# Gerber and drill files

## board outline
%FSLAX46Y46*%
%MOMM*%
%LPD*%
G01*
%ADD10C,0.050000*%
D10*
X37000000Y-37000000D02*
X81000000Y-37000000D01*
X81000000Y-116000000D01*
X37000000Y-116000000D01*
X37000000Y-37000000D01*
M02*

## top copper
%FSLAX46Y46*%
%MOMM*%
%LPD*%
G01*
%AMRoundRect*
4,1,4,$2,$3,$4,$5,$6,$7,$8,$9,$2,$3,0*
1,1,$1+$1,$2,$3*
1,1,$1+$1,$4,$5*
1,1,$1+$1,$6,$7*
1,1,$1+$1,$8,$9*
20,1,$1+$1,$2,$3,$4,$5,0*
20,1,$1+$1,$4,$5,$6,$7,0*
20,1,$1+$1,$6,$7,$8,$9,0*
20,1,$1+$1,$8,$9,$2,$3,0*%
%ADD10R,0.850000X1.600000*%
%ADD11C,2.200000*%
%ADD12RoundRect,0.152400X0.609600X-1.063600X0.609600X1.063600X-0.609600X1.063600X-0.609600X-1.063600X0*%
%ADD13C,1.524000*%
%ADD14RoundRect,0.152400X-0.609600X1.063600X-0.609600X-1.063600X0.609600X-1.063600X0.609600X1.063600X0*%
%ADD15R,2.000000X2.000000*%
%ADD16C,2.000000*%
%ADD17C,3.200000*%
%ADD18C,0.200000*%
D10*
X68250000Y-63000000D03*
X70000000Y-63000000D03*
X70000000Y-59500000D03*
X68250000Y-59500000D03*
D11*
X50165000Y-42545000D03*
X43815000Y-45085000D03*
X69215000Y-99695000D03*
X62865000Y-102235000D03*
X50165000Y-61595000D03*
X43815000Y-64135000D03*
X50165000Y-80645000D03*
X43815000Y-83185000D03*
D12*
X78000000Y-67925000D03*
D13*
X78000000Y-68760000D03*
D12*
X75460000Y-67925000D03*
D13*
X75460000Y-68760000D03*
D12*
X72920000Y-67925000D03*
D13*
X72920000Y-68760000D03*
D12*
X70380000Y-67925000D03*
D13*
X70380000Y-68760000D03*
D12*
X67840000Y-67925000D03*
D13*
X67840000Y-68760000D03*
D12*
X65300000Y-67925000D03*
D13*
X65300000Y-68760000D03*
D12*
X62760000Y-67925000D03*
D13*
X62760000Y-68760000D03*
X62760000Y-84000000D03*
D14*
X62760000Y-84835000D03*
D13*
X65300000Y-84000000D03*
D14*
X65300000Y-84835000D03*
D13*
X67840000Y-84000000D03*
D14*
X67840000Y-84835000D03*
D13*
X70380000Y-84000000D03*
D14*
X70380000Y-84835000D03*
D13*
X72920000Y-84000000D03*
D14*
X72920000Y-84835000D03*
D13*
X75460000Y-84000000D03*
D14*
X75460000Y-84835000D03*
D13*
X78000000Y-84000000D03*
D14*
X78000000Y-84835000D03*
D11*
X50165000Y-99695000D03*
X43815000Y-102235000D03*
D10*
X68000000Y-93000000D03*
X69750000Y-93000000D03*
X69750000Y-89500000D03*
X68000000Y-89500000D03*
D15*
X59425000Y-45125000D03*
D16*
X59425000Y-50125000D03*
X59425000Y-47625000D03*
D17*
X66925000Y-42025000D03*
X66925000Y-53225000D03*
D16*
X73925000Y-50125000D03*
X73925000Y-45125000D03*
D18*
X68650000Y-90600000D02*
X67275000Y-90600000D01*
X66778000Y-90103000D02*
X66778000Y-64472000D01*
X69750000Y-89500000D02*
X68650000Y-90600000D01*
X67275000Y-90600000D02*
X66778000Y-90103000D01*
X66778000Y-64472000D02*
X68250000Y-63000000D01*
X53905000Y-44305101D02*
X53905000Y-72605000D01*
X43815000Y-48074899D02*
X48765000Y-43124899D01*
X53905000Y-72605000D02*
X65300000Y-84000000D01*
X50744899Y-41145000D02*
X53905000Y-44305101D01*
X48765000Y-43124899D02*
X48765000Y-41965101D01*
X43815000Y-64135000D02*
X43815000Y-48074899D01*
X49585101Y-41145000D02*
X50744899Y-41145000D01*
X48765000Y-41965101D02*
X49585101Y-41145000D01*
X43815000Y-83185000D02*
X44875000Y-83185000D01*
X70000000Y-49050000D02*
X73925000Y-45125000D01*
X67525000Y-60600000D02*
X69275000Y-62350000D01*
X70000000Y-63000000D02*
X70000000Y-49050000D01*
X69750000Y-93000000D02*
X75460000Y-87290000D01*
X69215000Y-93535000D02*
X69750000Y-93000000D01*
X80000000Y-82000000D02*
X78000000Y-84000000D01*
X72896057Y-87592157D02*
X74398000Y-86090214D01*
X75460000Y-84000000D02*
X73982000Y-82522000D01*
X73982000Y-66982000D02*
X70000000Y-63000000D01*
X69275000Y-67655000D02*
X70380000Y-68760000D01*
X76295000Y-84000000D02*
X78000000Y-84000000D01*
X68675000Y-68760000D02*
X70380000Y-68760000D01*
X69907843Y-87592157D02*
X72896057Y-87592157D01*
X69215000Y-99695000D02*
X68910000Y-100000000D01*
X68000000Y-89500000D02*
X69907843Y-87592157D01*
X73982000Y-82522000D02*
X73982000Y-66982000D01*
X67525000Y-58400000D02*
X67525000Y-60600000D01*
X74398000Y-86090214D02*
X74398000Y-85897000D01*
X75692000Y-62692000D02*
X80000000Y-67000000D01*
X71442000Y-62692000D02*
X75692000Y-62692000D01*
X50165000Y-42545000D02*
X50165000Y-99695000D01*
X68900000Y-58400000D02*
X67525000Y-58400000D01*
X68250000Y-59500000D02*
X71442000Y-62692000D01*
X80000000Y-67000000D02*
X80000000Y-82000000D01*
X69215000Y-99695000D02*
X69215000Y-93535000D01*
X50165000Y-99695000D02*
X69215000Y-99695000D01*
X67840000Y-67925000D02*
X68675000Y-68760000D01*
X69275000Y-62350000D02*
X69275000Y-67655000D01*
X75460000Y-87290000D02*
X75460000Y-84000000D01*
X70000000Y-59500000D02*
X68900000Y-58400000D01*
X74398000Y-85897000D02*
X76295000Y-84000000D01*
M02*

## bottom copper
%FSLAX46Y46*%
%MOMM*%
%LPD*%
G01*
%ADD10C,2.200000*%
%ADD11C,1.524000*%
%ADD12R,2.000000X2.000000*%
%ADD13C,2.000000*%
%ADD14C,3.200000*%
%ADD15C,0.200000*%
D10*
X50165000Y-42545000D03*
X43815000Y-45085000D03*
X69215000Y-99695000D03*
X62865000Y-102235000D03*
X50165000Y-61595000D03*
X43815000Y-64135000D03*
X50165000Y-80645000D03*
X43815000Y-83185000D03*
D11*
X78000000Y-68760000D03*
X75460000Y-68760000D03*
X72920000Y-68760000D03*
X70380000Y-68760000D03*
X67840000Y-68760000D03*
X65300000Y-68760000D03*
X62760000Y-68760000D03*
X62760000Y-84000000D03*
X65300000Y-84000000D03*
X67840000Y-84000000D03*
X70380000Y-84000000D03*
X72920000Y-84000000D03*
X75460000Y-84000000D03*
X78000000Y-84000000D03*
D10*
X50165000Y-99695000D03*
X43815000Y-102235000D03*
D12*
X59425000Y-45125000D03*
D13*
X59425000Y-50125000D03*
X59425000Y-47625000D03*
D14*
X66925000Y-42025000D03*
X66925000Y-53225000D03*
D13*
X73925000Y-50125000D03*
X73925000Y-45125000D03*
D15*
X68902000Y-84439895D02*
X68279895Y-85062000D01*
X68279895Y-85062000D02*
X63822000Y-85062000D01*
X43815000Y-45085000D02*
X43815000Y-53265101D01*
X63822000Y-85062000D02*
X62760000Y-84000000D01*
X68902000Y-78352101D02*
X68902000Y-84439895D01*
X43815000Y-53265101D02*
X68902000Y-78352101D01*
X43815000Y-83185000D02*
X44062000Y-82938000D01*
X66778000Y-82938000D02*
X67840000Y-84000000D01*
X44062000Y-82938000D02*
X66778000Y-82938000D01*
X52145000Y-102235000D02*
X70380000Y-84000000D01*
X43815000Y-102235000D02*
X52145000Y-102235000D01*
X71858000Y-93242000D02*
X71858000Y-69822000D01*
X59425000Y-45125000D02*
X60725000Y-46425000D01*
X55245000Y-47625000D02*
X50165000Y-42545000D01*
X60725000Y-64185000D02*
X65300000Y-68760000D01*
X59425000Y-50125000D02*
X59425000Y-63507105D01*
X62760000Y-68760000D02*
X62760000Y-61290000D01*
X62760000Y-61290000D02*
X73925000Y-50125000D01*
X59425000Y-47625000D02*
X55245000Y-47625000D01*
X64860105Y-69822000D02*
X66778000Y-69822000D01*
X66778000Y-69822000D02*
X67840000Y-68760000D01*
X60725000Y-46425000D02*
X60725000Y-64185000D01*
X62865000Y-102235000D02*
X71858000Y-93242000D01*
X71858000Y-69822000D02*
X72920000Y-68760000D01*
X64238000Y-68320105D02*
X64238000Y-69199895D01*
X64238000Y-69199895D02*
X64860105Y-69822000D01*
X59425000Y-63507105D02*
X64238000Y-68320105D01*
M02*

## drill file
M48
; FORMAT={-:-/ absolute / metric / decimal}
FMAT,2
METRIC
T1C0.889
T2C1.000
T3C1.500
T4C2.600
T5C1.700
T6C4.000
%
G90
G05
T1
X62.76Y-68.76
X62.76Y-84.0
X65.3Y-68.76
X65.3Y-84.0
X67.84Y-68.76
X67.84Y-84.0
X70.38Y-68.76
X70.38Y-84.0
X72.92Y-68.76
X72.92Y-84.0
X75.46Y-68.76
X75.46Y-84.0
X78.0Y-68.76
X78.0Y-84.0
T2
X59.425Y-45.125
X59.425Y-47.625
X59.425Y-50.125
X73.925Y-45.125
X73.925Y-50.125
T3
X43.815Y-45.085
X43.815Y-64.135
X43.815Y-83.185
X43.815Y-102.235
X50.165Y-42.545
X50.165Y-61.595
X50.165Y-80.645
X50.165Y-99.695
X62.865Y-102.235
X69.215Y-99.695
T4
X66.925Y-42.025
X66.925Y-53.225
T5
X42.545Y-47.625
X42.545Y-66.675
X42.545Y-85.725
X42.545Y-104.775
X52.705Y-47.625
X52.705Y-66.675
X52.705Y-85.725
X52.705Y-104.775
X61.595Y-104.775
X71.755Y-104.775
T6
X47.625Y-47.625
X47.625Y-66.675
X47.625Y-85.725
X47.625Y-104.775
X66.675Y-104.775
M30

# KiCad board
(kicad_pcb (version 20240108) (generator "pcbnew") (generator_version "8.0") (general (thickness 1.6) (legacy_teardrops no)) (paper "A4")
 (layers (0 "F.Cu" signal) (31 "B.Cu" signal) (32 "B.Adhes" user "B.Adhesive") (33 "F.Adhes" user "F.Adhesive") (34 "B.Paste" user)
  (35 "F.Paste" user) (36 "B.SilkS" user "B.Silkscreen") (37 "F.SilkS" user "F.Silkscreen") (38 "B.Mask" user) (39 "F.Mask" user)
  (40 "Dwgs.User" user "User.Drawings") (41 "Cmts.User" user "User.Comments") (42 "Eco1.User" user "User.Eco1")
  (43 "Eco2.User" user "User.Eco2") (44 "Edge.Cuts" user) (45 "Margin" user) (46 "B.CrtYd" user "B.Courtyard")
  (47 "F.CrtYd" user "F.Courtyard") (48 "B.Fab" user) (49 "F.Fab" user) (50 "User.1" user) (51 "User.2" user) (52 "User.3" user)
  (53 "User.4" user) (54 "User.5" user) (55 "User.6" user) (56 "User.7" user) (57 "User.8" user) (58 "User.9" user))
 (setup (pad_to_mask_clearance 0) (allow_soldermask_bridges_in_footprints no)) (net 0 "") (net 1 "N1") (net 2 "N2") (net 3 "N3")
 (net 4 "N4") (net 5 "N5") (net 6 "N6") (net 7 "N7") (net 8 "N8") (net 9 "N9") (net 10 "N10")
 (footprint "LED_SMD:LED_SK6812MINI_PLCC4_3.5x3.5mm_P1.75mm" (layer "F.Cu") (at 69.125 61.25 90)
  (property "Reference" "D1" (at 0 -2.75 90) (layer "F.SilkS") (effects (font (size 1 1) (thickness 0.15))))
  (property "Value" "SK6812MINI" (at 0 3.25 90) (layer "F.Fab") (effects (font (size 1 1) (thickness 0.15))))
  (pad "1" smd rect (at -1.75 -0.875 90) (size 1.6 0.85) (layers "F.Cu" "F.Paste" "F.Mask") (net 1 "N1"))
  (pad "2" smd rect (at -1.75 0.875 90) (size 1.6 0.85) (layers "F.Cu" "F.Paste" "F.Mask") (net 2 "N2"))
  (pad "3" smd rect (at 1.75 0.875 90) (size 1.6 0.85) (layers "F.Cu" "F.Paste" "F.Mask") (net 2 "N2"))
  (pad "4" smd rect (at 1.75 -0.875 90) (size 1.6 0.85) (layers "F.Cu" "F.Paste" "F.Mask") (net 2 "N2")))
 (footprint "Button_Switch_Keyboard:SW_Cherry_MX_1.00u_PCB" (layer "F.Cu") (at 50.165 42.545)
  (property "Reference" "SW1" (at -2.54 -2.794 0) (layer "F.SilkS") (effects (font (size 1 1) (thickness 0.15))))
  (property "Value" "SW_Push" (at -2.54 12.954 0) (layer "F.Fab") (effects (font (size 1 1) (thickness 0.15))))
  (pad "" np_thru_hole circle (at -7.62 5.08) (size 1.7 1.7) (drill 1.7) (layers "*.Cu" "*.Mask"))
  (pad "" np_thru_hole circle (at -2.54 5.08) (size 4 4) (drill 4) (layers "*.Cu" "*.Mask"))
  (pad "" np_thru_hole circle (at 2.54 5.08) (size 1.7 1.7) (drill 1.7) (layers "*.Cu" "*.Mask"))
  (pad "1" thru_hole circle (at 0 0) (size 2.2 2.2) (drill 1.5) (layers "*.Cu" "*.Mask") (remove_unused_layers no) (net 2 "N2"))
  (pad "2" thru_hole circle (at -6.35 2.54) (size 2.2 2.2) (drill 1.5) (layers "*.Cu" "*.Mask") (remove_unused_layers no) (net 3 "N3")))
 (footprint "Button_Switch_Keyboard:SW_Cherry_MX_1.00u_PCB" (layer "F.Cu") (at 69.215 99.695)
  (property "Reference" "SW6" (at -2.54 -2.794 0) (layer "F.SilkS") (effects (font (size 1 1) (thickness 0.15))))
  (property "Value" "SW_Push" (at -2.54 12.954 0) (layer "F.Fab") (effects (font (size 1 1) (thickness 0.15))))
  (pad "" np_thru_hole circle (at -7.62 5.08) (size 1.7 1.7) (drill 1.7) (layers "*.Cu" "*.Mask"))
  (pad "" np_thru_hole circle (at -2.54 5.08) (size 4 4) (drill 4) (layers "*.Cu" "*.Mask"))
  (pad "" np_thru_hole circle (at 2.54 5.08) (size 1.7 1.7) (drill 1.7) (layers "*.Cu" "*.Mask"))
  (pad "1" thru_hole circle (at 0 0) (size 2.2 2.2) (drill 1.5) (layers "*.Cu" "*.Mask") (remove_unused_layers no) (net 2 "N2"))
  (pad "2" thru_hole circle (at -6.35 2.54) (size 2.2 2.2) (drill 1.5) (layers "*.Cu" "*.Mask") (remove_unused_layers no) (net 2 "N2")))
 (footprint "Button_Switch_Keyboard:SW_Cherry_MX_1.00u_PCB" (layer "F.Cu") (at 50.165 61.595)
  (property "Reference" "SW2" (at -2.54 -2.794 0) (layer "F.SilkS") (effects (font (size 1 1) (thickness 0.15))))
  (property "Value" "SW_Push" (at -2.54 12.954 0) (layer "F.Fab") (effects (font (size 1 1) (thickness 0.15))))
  (pad "" np_thru_hole circle (at -7.62 5.08) (size 1.7 1.7) (drill 1.7) (layers "*.Cu" "*.Mask"))
  (pad "" np_thru_hole circle (at -2.54 5.08) (size 4 4) (drill 4) (layers "*.Cu" "*.Mask"))
  (pad "" np_thru_hole circle (at 2.54 5.08) (size 1.7 1.7) (drill 1.7) (layers "*.Cu" "*.Mask"))
  (pad "1" thru_hole circle (at 0 0) (size 2.2 2.2) (drill 1.5) (layers "*.Cu" "*.Mask") (remove_unused_layers no) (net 2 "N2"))
  (pad "2" thru_hole circle (at -6.35 2.54) (size 2.2 2.2) (drill 1.5) (layers "*.Cu" "*.Mask") (remove_unused_layers no) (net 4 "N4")))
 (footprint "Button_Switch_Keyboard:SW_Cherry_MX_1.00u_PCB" (layer "F.Cu") (at 50.165 80.645)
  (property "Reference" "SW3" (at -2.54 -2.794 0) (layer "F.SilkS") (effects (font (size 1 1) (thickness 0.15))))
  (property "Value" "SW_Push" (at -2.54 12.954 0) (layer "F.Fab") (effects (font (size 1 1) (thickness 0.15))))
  (pad "" np_thru_hole circle (at -7.62 5.08) (size 1.7 1.7) (drill 1.7) (layers "*.Cu" "*.Mask"))
  (pad "" np_thru_hole circle (at -2.54 5.08) (size 4 4) (drill 4) (layers "*.Cu" "*.Mask"))
  (pad "" np_thru_hole circle (at 2.54 5.08) (size 1.7 1.7) (drill 1.7) (layers "*.Cu" "*.Mask"))
  (pad "1" thru_hole circle (at 0 0) (size 2.2 2.2) (drill 1.5) (layers "*.Cu" "*.Mask") (remove_unused_layers no) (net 2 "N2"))
  (pad "2" thru_hole circle (at -6.35 2.54) (size 2.2 2.2) (drill 1.5) (layers "*.Cu" "*.Mask") (remove_unused_layers no) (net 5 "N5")))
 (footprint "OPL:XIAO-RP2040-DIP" (layer "F.Cu") (at 70.38 76.38 -90)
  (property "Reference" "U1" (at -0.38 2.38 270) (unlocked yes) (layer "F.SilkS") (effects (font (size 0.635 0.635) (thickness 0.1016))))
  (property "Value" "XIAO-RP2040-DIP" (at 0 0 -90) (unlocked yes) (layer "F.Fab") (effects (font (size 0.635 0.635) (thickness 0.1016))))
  (pad "1" smd roundrect (at -8.455 -7.62 90) (size 2.432 1.524) (layers "F.Cu" "F.Mask") (roundrect_rratio 0.1) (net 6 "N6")
   (thermal_bridge_angle 45))
  (pad "1" thru_hole circle (at -7.62 -7.62 90) (size 1.524 1.524) (drill 0.889) (layers "*.Cu" "*.Mask") (remove_unused_layers no)
   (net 6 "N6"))
  (pad "2" smd roundrect (at -8.455 -5.08 90) (size 2.432 1.524) (layers "F.Cu" "F.Mask") (roundrect_rratio 0.1) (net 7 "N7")
   (thermal_bridge_angle 45))
  (pad "2" thru_hole circle (at -7.62 -5.08 90) (size 1.524 1.524) (drill 0.889) (layers "*.Cu" "*.Mask") (remove_unused_layers no)
   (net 7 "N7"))
  (pad "3" smd roundrect (at -8.455 -2.54 90) (size 2.432 1.524) (layers "F.Cu" "F.Mask") (roundrect_rratio 0.1) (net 2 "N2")
   (thermal_bridge_angle 45))
  (pad "3" thru_hole circle (at -7.62 -2.54 90) (size 1.524 1.524) (drill 0.889) (layers "*.Cu" "*.Mask") (remove_unused_layers no)
   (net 2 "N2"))
  (pad "4" smd roundrect (at -8.455 0 90) (size 2.432 1.524) (layers "F.Cu" "F.Mask") (roundrect_rratio 0.1) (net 2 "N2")
   (thermal_bridge_angle 45))
  (pad "4" thru_hole circle (at -7.62 0 90) (size 1.524 1.524) (drill 0.889) (layers "*.Cu" "*.Mask") (remove_unused_layers no) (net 2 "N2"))
  (pad "5" smd roundrect (at -8.455 2.54 90) (size 2.432 1.524) (layers "F.Cu" "F.Mask") (roundrect_rratio 0.1) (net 2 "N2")
   (thermal_bridge_angle 45))
  (pad "5" thru_hole circle (at -7.62 2.54 90) (size 1.524 1.524) (drill 0.889) (layers "*.Cu" "*.Mask") (remove_unused_layers no)
   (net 2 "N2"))
  (pad "6" smd roundrect (at -8.455 5.08 90) (size 2.432 1.524) (layers "F.Cu" "F.Mask") (roundrect_rratio 0.1) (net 2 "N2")
   (thermal_bridge_angle 45))
  (pad "6" thru_hole circle (at -7.62 5.08 90) (size 1.524 1.524) (drill 0.889) (layers "*.Cu" "*.Mask") (remove_unused_layers no)
   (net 2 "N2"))
  (pad "7" smd roundrect (at -8.455 7.62 90) (size 2.432 1.524) (layers "F.Cu" "F.Mask") (roundrect_rratio 0.1) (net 2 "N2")
   (thermal_bridge_angle 45))
  (pad "7" thru_hole circle (at -7.62 7.62 90) (size 1.524 1.524) (drill 0.889) (layers "*.Cu" "*.Mask") (remove_unused_layers no)
   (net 2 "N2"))
  (pad "8" thru_hole circle (at 7.62 7.62 270) (size 1.524 1.524) (drill 0.889) (layers "*.Cu" "*.Mask") (remove_unused_layers no)
   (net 3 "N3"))
  (pad "8" smd roundrect (at 8.455 7.62 270) (size 2.432 1.524) (layers "F.Cu" "F.Mask") (roundrect_rratio 0.1) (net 3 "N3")
   (thermal_bridge_angle 45))
  (pad "9" thru_hole circle (at 7.62 5.08 270) (size 1.524 1.524) (drill 0.889) (layers "*.Cu" "*.Mask") (remove_unused_layers no)
   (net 4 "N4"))
  (pad "9" smd roundrect (at 8.455 5.08 270) (size 2.432 1.524) (layers "F.Cu" "F.Mask") (roundrect_rratio 0.1) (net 4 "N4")
   (thermal_bridge_angle 45))
  (pad "10" thru_hole circle (at 7.62 2.54 270) (size 1.524 1.524) (drill 0.889) (layers "*.Cu" "*.Mask") (remove_unused_layers no)
   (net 5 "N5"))
  (pad "10" smd roundrect (at 8.455 2.54 270) (size 2.432 1.524) (layers "F.Cu" "F.Mask") (roundrect_rratio 0.1) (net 5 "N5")
   (thermal_bridge_angle 45))
  (pad "11" thru_hole circle (at 7.62 0 270) (size 1.524 1.524) (drill 0.889) (layers "*.Cu" "*.Mask") (remove_unused_layers no)
   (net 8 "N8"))
  (pad "11" smd roundrect (at 8.455 0 270) (size 2.432 1.524) (layers "F.Cu" "F.Mask") (roundrect_rratio 0.1) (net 8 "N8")
   (thermal_bridge_angle 45))
  (pad "12" thru_hole circle (at 7.62 -2.54 270) (size 1.524 1.524) (drill 0.889) (layers "*.Cu" "*.Mask") (remove_unused_layers no)
   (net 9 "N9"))
  (pad "12" smd roundrect (at 8.455 -2.54 270) (size 2.432 1.524) (layers "F.Cu" "F.Mask") (roundrect_rratio 0.1) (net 9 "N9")
   (thermal_bridge_angle 45))
  (pad "13" thru_hole circle (at 7.62 -5.08 270) (size 1.524 1.524) (drill 0.889) (layers "*.Cu" "*.Mask") (remove_unused_layers no)
   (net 2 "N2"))
  (pad "13" smd roundrect (at 8.455 -5.08 270) (size 2.432 1.524) (layers "F.Cu" "F.Mask") (roundrect_rratio 0.1) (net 2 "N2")
   (thermal_bridge_angle 45))
  (pad "14" thru_hole circle (at 7.62 -7.62 270) (size 1.524 1.524) (drill 0.889) (layers "*.Cu" "*.Mask") (remove_unused_layers no)
   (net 2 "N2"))
  (pad "14" smd roundrect (at 8.455 -7.62 270) (size 2.432 1.524) (layers "F.Cu" "F.Mask") (roundrect_rratio 0.1) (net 2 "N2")
   (thermal_bridge_angle 45)))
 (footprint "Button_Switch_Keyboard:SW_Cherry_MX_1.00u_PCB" (layer "F.Cu") (at 50.165 99.695)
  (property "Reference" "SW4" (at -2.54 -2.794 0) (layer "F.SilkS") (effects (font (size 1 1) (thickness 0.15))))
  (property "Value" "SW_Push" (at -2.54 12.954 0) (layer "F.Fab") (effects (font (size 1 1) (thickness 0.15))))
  (pad "" np_thru_hole circle (at -7.62 5.08) (size 1.7 1.7) (drill 1.7) (layers "*.Cu" "*.Mask"))
  (pad "" np_thru_hole circle (at -2.54 5.08) (size 4 4) (drill 4) (layers "*.Cu" "*.Mask"))
  (pad "" np_thru_hole circle (at 2.54 5.08) (size 1.7 1.7) (drill 1.7) (layers "*.Cu" "*.Mask"))
  (pad "1" thru_hole circle (at 0 0) (size 2.2 2.2) (drill 1.5) (layers "*.Cu" "*.Mask") (remove_unused_layers no) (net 2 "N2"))
  (pad "2" thru_hole circle (at -6.35 2.54) (size 2.2 2.2) (drill 1.5) (layers "*.Cu" "*.Mask") (remove_unused_layers no) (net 8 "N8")))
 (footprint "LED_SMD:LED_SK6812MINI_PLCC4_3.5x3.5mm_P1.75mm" (layer "F.Cu") (at 68.875 91.25 90)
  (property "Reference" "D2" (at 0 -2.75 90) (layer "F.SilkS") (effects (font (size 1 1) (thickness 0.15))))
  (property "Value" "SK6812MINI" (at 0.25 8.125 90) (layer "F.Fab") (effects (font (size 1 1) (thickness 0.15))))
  (pad "1" smd rect (at -1.75 -0.875 90) (size 1.6 0.85) (layers "F.Cu" "F.Paste" "F.Mask") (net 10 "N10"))
  (pad "2" smd rect (at -1.75 0.875 90) (size 1.6 0.85) (layers "F.Cu" "F.Paste" "F.Mask") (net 2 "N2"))
  (pad "3" smd rect (at 1.75 0.875 90) (size 1.6 0.85) (layers "F.Cu" "F.Paste" "F.Mask") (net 1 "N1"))
  (pad "4" smd rect (at 1.75 -0.875 90) (size 1.6 0.85) (layers "F.Cu" "F.Paste" "F.Mask") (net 2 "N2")))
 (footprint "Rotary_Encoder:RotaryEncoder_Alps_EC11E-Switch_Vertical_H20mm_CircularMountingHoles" (layer "F.Cu") (at 59.425 45.125)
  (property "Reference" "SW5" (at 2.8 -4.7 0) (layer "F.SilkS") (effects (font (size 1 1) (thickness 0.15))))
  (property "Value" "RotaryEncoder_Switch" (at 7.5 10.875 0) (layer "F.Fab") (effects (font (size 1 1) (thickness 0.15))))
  (pad "A" thru_hole rect (at 0 0) (size 2 2) (drill 1) (layers "*.Cu" "*.Mask") (remove_unused_layers no) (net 2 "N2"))
  (pad "B" thru_hole circle (at 0 5) (size 2 2) (drill 1) (layers "*.Cu" "*.Mask") (remove_unused_layers no) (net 2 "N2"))
  (pad "C" thru_hole circle (at 0 2.5) (size 2 2) (drill 1) (layers "*.Cu" "*.Mask") (remove_unused_layers no) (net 2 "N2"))
  (pad "MP" thru_hole circle (at 7.5 -3.1) (size 3.2 3.2) (drill 2.6) (layers "*.Cu" "*.Mask") (remove_unused_layers no))
  (pad "MP" thru_hole circle (at 7.5 8.1) (size 3.2 3.2) (drill 2.6) (layers "*.Cu" "*.Mask") (remove_unused_layers no))
  (pad "S1" thru_hole circle (at 14.5 5) (size 2 2) (drill 1) (layers "*.Cu" "*.Mask") (remove_unused_layers no) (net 2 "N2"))
  (pad "S2" thru_hole circle (at 14.5 0) (size 2 2) (drill 1) (layers "*.Cu" "*.Mask") (remove_unused_layers no) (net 2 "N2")))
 (gr_rect (start 37 37) (end 81 116) (stroke (width 0.05) (type default)) (fill none) (layer "Edge.Cuts"))
 (segment (start 68.65 90.6) (end 67.275 90.6) (width 0.2) (layer "F.Cu") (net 1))
 (segment (start 66.778 90.103) (end 66.778 64.472) (width 0.2) (layer "F.Cu") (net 1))
 (segment (start 69.75 89.5) (end 68.65 90.6) (width 0.2) (layer "F.Cu") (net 1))
 (segment (start 67.275 90.6) (end 66.778 90.103) (width 0.2) (layer "F.Cu") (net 1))
 (segment (start 66.778 64.472) (end 68.25 63) (width 0.2) (layer "F.Cu") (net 1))
 (segment (start 68.902 84.439895) (end 68.279895 85.062) (width 0.2) (layer "B.Cu") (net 3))
 (segment (start 68.279895 85.062) (end 63.822 85.062) (width 0.2) (layer "B.Cu") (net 3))
 (segment (start 43.815 45.085) (end 43.815 53.265101) (width 0.2) (layer "B.Cu") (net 3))
 (segment (start 63.822 85.062) (end 62.76 84) (width 0.2) (layer "B.Cu") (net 3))
 (segment (start 68.902 78.352101) (end 68.902 84.439895) (width 0.2) (layer "B.Cu") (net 3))
 (segment (start 43.815 53.265101) (end 68.902 78.352101) (width 0.2) (layer "B.Cu") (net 3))
 (segment (start 53.905 44.305101) (end 53.905 72.605) (width 0.2) (layer "F.Cu") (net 4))
 (segment (start 43.815 48.074899) (end 48.765 43.124899) (width 0.2) (layer "F.Cu") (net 4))
 (segment (start 53.905 72.605) (end 65.3 84) (width 0.2) (layer "F.Cu") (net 4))
 (segment (start 50.744899 41.145) (end 53.905 44.305101) (width 0.2) (layer "F.Cu") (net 4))
 (segment (start 48.765 43.124899) (end 48.765 41.965101) (width 0.2) (layer "F.Cu") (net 4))
 (segment (start 43.815 64.135) (end 43.815 48.074899) (width 0.2) (layer "F.Cu") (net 4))
 (segment (start 49.585101 41.145) (end 50.744899 41.145) (width 0.2) (layer "F.Cu") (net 4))
 (segment (start 48.765 41.965101) (end 49.585101 41.145) (width 0.2) (layer "F.Cu") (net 4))
 (segment (start 43.815 83.185) (end 44.875 83.185) (width 0.2) (layer "F.Cu") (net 5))
 (segment (start 43.815 83.185) (end 44.062 82.938) (width 0.2) (layer "B.Cu") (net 5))
 (segment (start 66.778 82.938) (end 67.84 84) (width 0.2) (layer "B.Cu") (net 5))
 (segment (start 44.062 82.938) (end 66.778 82.938) (width 0.2) (layer "B.Cu") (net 5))
 (segment (start 52.145 102.235) (end 70.38 84) (width 0.2) (layer "B.Cu") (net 8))
 (segment (start 43.815 102.235) (end 52.145 102.235) (width 0.2) (layer "B.Cu") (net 8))
 (segment (start 70 49.05) (end 73.925 45.125) (width 0.2) (layer "F.Cu") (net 2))
 (segment (start 67.525 60.6) (end 69.275 62.35) (width 0.2) (layer "F.Cu") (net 2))
 (segment (start 70 63) (end 70 49.05) (width 0.2) (layer "F.Cu") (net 2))
 (segment (start 69.75 93) (end 75.46 87.29) (width 0.2) (layer "F.Cu") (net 2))
 (segment (start 69.215 93.535) (end 69.75 93) (width 0.2) (layer "F.Cu") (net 2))
 (segment (start 80 82) (end 78 84) (width 0.2) (layer "F.Cu") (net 2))
 (segment (start 72.896057 87.592157) (end 74.398 86.090214) (width 0.2) (layer "F.Cu") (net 2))
 (segment (start 75.46 84) (end 73.982 82.522) (width 0.2) (layer "F.Cu") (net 2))
 (segment (start 73.982 66.982) (end 70 63) (width 0.2) (layer "F.Cu") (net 2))
 (segment (start 69.275 67.655) (end 70.38 68.76) (width 0.2) (layer "F.Cu") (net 2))
 (segment (start 76.295 84) (end 78 84) (width 0.2) (layer "F.Cu") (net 2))
 (segment (start 68.675 68.76) (end 70.38 68.76) (width 0.2) (layer "F.Cu") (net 2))
 (segment (start 69.907843 87.592157) (end 72.896057 87.592157) (width 0.2) (layer "F.Cu") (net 2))
 (segment (start 69.215 99.695) (end 68.91 100) (width 0.2) (layer "F.Cu") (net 2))
 (segment (start 68 89.5) (end 69.907843 87.592157) (width 0.2) (layer "F.Cu") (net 2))
 (segment (start 73.982 82.522) (end 73.982 66.982) (width 0.2) (layer "F.Cu") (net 2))
 (segment (start 67.525 58.4) (end 67.525 60.6) (width 0.2) (layer "F.Cu") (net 2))
 (segment (start 74.398 86.090214) (end 74.398 85.897) (width 0.2) (layer "F.Cu") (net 2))
 (segment (start 75.692 62.692) (end 80 67) (width 0.2) (layer "F.Cu") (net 2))
 (segment (start 71.442 62.692) (end 75.692 62.692) (width 0.2) (layer "F.Cu") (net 2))
 (segment (start 50.165 42.545) (end 50.165 99.695) (width 0.2) (layer "F.Cu") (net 2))
 (segment (start 68.9 58.4) (end 67.525 58.4) (width 0.2) (layer "F.Cu") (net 2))
 (segment (start 68.25 59.5) (end 71.442 62.692) (width 0.2) (layer "F.Cu") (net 2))
 (segment (start 80 67) (end 80 82) (width 0.2) (layer "F.Cu") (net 2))
 (segment (start 69.215 99.695) (end 69.215 93.535) (width 0.2) (layer "F.Cu") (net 2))
 (segment (start 50.165 99.695) (end 69.215 99.695) (width 0.2) (layer "F.Cu") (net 2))
 (segment (start 67.84 67.925) (end 68.675 68.76) (width 0.2) (layer "F.Cu") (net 2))
 (segment (start 69.275 62.35) (end 69.275 67.655) (width 0.2) (layer "F.Cu") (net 2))
 (segment (start 75.46 87.29) (end 75.46 84) (width 0.2) (layer "F.Cu") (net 2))
 (segment (start 70 59.5) (end 68.9 58.4) (width 0.2) (layer "F.Cu") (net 2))
 (segment (start 74.398 85.897) (end 76.295 84) (width 0.2) (layer "F.Cu") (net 2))
 (segment (start 71.858 93.242) (end 71.858 69.822) (width 0.2) (layer "B.Cu") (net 2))
 (segment (start 59.425 45.125) (end 60.725 46.425) (width 0.2) (layer "B.Cu") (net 2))
 (segment (start 55.245 47.625) (end 50.165 42.545) (width 0.2) (layer "B.Cu") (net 2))
 (segment (start 60.725 64.185) (end 65.3 68.76) (width 0.2) (layer "B.Cu") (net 2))
 (segment (start 59.425 50.125) (end 59.425 63.507105) (width 0.2) (layer "B.Cu") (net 2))
 (segment (start 62.76 68.76) (end 62.76 61.29) (width 0.2) (layer "B.Cu") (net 2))
 (segment (start 62.76 61.29) (end 73.925 50.125) (width 0.2) (layer "B.Cu") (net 2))
 (segment (start 59.425 47.625) (end 55.245 47.625) (width 0.2) (layer "B.Cu") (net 2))
 (segment (start 64.860105 69.822) (end 66.778 69.822) (width 0.2) (layer "B.Cu") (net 2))
 (segment (start 66.778 69.822) (end 67.84 68.76) (width 0.2) (layer "B.Cu") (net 2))
 (segment (start 60.725 46.425) (end 60.725 64.185) (width 0.2) (layer "B.Cu") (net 2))
 (segment (start 62.865 102.235) (end 71.858 93.242) (width 0.2) (layer "B.Cu") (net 2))
 (segment (start 71.858 69.822) (end 72.92 68.76) (width 0.2) (layer "B.Cu") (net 2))
 (segment (start 64.238 68.320105) (end 64.238 69.199895) (width 0.2) (layer "B.Cu") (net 2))
 (segment (start 64.238 69.199895) (end 64.860105 69.822) (width 0.2) (layer "B.Cu") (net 2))
 (segment (start 59.425 63.507105) (end 64.238 68.320105) (width 0.2) (layer "B.Cu") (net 2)))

